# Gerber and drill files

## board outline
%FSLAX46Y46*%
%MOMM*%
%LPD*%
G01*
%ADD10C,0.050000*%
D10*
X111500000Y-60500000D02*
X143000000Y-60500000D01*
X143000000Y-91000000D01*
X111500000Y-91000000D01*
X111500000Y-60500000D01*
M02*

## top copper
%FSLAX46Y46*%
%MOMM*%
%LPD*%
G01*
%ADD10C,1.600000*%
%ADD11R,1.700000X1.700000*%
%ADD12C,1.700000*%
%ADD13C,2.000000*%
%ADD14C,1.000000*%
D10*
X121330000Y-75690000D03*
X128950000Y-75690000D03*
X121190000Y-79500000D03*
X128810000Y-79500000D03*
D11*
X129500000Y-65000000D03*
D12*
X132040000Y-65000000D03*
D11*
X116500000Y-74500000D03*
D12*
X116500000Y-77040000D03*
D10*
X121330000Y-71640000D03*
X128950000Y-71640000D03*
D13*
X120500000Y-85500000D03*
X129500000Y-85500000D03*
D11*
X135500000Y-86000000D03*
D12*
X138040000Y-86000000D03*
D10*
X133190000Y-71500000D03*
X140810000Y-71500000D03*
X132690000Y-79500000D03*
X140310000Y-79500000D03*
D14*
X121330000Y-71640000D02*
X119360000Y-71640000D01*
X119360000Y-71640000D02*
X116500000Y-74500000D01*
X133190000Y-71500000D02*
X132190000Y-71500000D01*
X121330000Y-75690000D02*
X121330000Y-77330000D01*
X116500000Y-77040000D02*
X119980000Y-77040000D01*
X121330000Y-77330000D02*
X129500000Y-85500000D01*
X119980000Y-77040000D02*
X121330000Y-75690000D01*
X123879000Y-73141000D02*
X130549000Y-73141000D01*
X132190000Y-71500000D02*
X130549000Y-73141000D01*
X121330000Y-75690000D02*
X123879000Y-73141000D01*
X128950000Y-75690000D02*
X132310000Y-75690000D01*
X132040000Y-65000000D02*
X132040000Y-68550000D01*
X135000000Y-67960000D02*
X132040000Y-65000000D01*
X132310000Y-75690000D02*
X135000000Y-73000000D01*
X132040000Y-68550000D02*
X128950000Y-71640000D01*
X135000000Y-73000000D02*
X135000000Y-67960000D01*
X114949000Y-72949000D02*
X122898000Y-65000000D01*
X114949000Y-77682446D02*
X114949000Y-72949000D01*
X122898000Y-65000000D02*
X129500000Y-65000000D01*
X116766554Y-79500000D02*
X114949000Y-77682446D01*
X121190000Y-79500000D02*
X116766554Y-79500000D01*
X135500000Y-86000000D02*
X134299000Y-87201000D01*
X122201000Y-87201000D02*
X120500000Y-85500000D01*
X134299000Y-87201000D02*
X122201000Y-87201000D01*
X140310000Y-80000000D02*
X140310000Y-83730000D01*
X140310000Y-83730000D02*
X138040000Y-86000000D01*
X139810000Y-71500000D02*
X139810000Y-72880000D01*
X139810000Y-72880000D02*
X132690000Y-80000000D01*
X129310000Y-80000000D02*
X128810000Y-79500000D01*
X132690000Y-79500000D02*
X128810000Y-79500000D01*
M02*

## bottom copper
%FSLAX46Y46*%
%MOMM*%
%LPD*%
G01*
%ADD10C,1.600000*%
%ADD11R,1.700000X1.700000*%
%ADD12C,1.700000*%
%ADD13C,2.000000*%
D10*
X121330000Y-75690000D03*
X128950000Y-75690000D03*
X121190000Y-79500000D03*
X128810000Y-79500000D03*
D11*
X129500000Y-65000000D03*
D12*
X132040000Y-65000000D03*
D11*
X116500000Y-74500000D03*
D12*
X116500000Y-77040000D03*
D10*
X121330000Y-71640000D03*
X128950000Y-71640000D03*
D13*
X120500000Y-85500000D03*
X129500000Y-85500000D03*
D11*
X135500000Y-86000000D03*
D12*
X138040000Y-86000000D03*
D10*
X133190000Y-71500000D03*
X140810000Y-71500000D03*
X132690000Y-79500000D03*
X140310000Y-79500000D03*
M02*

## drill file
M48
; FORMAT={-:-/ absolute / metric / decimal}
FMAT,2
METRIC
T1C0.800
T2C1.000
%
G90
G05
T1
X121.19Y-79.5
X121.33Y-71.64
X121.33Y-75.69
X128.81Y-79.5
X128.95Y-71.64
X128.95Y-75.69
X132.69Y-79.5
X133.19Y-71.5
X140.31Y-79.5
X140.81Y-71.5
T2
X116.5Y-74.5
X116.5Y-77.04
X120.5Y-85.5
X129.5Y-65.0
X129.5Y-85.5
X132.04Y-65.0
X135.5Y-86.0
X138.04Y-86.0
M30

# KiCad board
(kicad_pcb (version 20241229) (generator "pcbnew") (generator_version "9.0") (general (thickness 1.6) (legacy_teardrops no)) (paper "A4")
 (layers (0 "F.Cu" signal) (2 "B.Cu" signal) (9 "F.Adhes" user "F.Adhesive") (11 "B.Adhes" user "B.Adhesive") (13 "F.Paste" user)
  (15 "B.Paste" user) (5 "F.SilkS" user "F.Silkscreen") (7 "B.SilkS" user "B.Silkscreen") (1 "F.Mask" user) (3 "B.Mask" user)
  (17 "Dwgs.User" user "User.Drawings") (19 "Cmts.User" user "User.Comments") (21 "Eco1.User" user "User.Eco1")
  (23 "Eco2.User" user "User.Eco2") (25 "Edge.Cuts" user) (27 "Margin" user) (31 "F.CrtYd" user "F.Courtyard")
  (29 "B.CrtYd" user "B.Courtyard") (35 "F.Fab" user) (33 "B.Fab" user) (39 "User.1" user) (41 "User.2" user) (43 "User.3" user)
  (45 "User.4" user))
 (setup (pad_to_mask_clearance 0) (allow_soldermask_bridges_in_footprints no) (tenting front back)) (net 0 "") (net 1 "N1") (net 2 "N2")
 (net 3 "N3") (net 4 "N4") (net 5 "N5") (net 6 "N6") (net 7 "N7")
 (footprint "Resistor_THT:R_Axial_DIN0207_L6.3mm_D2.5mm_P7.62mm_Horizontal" (layer "F.Cu") (at 121.33 75.69)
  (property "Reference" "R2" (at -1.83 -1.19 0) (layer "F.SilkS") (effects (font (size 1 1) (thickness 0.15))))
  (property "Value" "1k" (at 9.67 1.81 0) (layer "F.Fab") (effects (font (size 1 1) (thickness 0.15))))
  (pad "1" thru_hole circle (at 0 0) (size 1.6 1.6) (drill 0.8) (layers "*.Cu" "*.Mask") (remove_unused_layers no) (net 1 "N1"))
  (pad "2" thru_hole circle (at 7.62 0) (size 1.6 1.6) (drill 0.8) (layers "*.Cu" "*.Mask") (remove_unused_layers no) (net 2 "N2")))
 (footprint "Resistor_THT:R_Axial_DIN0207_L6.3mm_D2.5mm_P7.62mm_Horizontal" (layer "F.Cu") (at 121.19 79.5)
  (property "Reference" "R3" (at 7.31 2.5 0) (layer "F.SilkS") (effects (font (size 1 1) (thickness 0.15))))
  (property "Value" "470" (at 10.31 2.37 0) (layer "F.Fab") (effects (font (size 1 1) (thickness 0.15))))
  (pad "1" thru_hole circle (at 0 0) (size 1.6 1.6) (drill 0.8) (layers "*.Cu" "*.Mask") (remove_unused_layers no) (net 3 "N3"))
  (pad "2" thru_hole circle (at 7.62 0) (size 1.6 1.6) (drill 0.8) (layers "*.Cu" "*.Mask") (remove_unused_layers no) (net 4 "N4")))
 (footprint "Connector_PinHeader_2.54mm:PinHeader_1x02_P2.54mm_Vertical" (layer "F.Cu") (at 129.5 65 90)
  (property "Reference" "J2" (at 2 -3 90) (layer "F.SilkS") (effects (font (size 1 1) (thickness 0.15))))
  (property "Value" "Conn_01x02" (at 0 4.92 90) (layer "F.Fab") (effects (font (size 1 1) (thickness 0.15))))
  (pad "1" thru_hole rect (at 0 0 90) (size 1.7 1.7) (drill 1) (layers "*.Cu" "*.Mask") (remove_unused_layers no) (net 3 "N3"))
  (pad "2" thru_hole circle (at 0 2.54 90) (size 1.7 1.7) (drill 1) (layers "*.Cu" "*.Mask") (remove_unused_layers no) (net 2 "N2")))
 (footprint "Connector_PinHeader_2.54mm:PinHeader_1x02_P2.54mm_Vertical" (layer "F.Cu") (at 116.5 74.5)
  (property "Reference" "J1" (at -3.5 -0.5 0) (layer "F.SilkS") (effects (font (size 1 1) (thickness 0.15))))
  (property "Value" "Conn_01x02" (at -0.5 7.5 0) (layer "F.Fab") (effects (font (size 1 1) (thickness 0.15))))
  (pad "1" thru_hole rect (at 0 0) (size 1.7 1.7) (drill 1) (layers "*.Cu" "*.Mask") (remove_unused_layers no) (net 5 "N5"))
  (pad "2" thru_hole circle (at 0 2.54) (size 1.7 1.7) (drill 1) (layers "*.Cu" "*.Mask") (remove_unused_layers no) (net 1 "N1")))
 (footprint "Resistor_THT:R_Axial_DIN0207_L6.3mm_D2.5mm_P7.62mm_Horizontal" (layer "F.Cu") (at 121.33 71.64)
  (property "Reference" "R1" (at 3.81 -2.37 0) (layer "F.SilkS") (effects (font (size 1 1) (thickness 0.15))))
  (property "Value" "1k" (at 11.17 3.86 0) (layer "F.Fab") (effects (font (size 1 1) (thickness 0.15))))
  (pad "1" thru_hole circle (at 0 0) (size 1.6 1.6) (drill 0.8) (layers "*.Cu" "*.Mask") (remove_unused_layers no) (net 5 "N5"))
  (pad "2" thru_hole circle (at 7.62 0) (size 1.6 1.6) (drill 0.8) (layers "*.Cu" "*.Mask") (remove_unused_layers no) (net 2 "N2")))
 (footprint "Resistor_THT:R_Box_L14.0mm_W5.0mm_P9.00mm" (layer "F.Cu") (at 120.5 85.5)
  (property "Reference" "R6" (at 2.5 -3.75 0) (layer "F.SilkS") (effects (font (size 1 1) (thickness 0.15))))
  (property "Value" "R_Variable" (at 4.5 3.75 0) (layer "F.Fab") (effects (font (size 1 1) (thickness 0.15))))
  (pad "1" thru_hole circle (at 0 0) (size 2 2) (drill 1) (layers "*.Cu" "*.Mask") (remove_unused_layers no) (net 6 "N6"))
  (pad "2" thru_hole circle (at 9 0) (size 2 2) (drill 1) (layers "*.Cu" "*.Mask") (remove_unused_layers no) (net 1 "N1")))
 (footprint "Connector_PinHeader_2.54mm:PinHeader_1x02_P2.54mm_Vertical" (layer "F.Cu") (at 135.5 86 90)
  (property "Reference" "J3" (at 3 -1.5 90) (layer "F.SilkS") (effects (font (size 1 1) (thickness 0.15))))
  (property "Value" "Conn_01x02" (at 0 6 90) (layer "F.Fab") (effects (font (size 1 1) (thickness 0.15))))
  (pad "1" thru_hole rect (at 0 0 90) (size 1.7 1.7) (drill 1) (layers "*.Cu" "*.Mask") (remove_unused_layers no) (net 6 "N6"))
  (pad "2" thru_hole circle (at 0 2.54 90) (size 1.7 1.7) (drill 1) (layers "*.Cu" "*.Mask") (remove_unused_layers no) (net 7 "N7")))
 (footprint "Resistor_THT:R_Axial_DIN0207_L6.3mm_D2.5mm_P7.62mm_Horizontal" (layer "F.Cu") (at 133.19 71.5)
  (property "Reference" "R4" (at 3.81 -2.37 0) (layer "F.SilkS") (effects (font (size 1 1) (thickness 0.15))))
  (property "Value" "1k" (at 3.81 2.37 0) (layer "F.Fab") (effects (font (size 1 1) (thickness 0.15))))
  (pad "1" thru_hole circle (at 0 0) (size 1.6 1.6) (drill 0.8) (layers "*.Cu" "*.Mask") (remove_unused_layers no) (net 1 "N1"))
  (pad "2" thru_hole circle (at 7.62 0) (size 1.6 1.6) (drill 0.8) (layers "*.Cu" "*.Mask") (remove_unused_layers no) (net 4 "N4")))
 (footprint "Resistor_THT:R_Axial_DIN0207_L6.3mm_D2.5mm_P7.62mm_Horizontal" (layer "F.Cu") (at 132.69 79.5)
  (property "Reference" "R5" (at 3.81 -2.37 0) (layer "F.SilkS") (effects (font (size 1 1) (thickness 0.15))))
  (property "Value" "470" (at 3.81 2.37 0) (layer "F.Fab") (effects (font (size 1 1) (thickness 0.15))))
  (pad "1" thru_hole circle (at 0 0) (size 1.6 1.6) (drill 0.8) (layers "*.Cu" "*.Mask") (remove_unused_layers no) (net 4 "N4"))
  (pad "2" thru_hole circle (at 7.62 0) (size 1.6 1.6) (drill 0.8) (layers "*.Cu" "*.Mask") (remove_unused_layers no) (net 7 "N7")))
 (gr_rect (start 111.5 60.5) (end 143 91) (stroke (width 0.05) (type default)) (fill no) (layer "Edge.Cuts"))
 (segment (start 121.33 71.64) (end 119.36 71.64) (width 1) (layer "F.Cu") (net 5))
 (segment (start 119.36 71.64) (end 116.5 74.5) (width 1) (layer "F.Cu") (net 5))
 (segment (start 133.19 71.5) (end 132.19 71.5) (width 1) (layer "F.Cu") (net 1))
 (segment (start 121.33 75.69) (end 121.33 77.33) (width 1) (layer "F.Cu") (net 1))
 (segment (start 116.5 77.04) (end 119.98 77.04) (width 1) (layer "F.Cu") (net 1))
 (segment (start 121.33 77.33) (end 129.5 85.5) (width 1) (layer "F.Cu") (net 1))
 (segment (start 119.98 77.04) (end 121.33 75.69) (width 1) (layer "F.Cu") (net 1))
 (segment (start 123.879 73.141) (end 130.549 73.141) (width 1) (layer "F.Cu") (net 1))
 (segment (start 132.19 71.5) (end 130.549 73.141) (width 1) (layer "F.Cu") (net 1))
 (segment (start 121.33 75.69) (end 123.879 73.141) (width 1) (layer "F.Cu") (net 1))
 (segment (start 128.95 75.69) (end 132.31 75.69) (width 1) (layer "F.Cu") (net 2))
 (segment (start 132.04 65) (end 132.04 68.55) (width 1) (layer "F.Cu") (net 2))
 (segment (start 135 67.96) (end 132.04 65) (width 1) (layer "F.Cu") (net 2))
 (segment (start 132.31 75.69) (end 135 73) (width 1) (layer "F.Cu") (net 2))
 (segment (start 132.04 68.55) (end 128.95 71.64) (width 1) (layer "F.Cu") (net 2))
 (segment (start 135 73) (end 135 67.96) (width 1) (layer "F.Cu") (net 2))
 (segment (start 114.949 72.949) (end 122.898 65) (width 1) (layer "F.Cu") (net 3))
 (segment (start 114.949 77.682446) (end 114.949 72.949) (width 1) (layer "F.Cu") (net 3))
 (segment (start 122.898 65) (end 129.5 65) (width 1) (layer "F.Cu") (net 3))
 (segment (start 116.766554 79.5) (end 114.949 77.682446) (width 1) (layer "F.Cu") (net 3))
 (segment (start 121.19 79.5) (end 116.766554 79.5) (width 1) (layer "F.Cu") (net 3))
 (segment (start 135.5 86) (end 134.299 87.201) (width 1) (layer "F.Cu") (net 6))
 (segment (start 122.201 87.201) (end 120.5 85.5) (width 1) (layer "F.Cu") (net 6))
 (segment (start 134.299 87.201) (end 122.201 87.201) (width 1) (layer "F.Cu") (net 6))
 (segment (start 140.31 80) (end 140.31 83.73) (width 1) (layer "F.Cu") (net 7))
 (segment (start 140.31 83.73) (end 138.04 86) (width 1) (layer "F.Cu") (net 7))
 (segment (start 139.81 71.5) (end 139.81 72.88) (width 1) (layer "F.Cu") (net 4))
 (segment (start 139.81 72.88) (end 132.69 80) (width 1) (layer "F.Cu") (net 4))
 (segment (start 129.31 80) (end 128.81 79.5) (width 1) (layer "F.Cu") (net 4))
 (segment (start 132.69 79.5) (end 128.81 79.5) (width 1) (layer "F.Cu") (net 4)))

